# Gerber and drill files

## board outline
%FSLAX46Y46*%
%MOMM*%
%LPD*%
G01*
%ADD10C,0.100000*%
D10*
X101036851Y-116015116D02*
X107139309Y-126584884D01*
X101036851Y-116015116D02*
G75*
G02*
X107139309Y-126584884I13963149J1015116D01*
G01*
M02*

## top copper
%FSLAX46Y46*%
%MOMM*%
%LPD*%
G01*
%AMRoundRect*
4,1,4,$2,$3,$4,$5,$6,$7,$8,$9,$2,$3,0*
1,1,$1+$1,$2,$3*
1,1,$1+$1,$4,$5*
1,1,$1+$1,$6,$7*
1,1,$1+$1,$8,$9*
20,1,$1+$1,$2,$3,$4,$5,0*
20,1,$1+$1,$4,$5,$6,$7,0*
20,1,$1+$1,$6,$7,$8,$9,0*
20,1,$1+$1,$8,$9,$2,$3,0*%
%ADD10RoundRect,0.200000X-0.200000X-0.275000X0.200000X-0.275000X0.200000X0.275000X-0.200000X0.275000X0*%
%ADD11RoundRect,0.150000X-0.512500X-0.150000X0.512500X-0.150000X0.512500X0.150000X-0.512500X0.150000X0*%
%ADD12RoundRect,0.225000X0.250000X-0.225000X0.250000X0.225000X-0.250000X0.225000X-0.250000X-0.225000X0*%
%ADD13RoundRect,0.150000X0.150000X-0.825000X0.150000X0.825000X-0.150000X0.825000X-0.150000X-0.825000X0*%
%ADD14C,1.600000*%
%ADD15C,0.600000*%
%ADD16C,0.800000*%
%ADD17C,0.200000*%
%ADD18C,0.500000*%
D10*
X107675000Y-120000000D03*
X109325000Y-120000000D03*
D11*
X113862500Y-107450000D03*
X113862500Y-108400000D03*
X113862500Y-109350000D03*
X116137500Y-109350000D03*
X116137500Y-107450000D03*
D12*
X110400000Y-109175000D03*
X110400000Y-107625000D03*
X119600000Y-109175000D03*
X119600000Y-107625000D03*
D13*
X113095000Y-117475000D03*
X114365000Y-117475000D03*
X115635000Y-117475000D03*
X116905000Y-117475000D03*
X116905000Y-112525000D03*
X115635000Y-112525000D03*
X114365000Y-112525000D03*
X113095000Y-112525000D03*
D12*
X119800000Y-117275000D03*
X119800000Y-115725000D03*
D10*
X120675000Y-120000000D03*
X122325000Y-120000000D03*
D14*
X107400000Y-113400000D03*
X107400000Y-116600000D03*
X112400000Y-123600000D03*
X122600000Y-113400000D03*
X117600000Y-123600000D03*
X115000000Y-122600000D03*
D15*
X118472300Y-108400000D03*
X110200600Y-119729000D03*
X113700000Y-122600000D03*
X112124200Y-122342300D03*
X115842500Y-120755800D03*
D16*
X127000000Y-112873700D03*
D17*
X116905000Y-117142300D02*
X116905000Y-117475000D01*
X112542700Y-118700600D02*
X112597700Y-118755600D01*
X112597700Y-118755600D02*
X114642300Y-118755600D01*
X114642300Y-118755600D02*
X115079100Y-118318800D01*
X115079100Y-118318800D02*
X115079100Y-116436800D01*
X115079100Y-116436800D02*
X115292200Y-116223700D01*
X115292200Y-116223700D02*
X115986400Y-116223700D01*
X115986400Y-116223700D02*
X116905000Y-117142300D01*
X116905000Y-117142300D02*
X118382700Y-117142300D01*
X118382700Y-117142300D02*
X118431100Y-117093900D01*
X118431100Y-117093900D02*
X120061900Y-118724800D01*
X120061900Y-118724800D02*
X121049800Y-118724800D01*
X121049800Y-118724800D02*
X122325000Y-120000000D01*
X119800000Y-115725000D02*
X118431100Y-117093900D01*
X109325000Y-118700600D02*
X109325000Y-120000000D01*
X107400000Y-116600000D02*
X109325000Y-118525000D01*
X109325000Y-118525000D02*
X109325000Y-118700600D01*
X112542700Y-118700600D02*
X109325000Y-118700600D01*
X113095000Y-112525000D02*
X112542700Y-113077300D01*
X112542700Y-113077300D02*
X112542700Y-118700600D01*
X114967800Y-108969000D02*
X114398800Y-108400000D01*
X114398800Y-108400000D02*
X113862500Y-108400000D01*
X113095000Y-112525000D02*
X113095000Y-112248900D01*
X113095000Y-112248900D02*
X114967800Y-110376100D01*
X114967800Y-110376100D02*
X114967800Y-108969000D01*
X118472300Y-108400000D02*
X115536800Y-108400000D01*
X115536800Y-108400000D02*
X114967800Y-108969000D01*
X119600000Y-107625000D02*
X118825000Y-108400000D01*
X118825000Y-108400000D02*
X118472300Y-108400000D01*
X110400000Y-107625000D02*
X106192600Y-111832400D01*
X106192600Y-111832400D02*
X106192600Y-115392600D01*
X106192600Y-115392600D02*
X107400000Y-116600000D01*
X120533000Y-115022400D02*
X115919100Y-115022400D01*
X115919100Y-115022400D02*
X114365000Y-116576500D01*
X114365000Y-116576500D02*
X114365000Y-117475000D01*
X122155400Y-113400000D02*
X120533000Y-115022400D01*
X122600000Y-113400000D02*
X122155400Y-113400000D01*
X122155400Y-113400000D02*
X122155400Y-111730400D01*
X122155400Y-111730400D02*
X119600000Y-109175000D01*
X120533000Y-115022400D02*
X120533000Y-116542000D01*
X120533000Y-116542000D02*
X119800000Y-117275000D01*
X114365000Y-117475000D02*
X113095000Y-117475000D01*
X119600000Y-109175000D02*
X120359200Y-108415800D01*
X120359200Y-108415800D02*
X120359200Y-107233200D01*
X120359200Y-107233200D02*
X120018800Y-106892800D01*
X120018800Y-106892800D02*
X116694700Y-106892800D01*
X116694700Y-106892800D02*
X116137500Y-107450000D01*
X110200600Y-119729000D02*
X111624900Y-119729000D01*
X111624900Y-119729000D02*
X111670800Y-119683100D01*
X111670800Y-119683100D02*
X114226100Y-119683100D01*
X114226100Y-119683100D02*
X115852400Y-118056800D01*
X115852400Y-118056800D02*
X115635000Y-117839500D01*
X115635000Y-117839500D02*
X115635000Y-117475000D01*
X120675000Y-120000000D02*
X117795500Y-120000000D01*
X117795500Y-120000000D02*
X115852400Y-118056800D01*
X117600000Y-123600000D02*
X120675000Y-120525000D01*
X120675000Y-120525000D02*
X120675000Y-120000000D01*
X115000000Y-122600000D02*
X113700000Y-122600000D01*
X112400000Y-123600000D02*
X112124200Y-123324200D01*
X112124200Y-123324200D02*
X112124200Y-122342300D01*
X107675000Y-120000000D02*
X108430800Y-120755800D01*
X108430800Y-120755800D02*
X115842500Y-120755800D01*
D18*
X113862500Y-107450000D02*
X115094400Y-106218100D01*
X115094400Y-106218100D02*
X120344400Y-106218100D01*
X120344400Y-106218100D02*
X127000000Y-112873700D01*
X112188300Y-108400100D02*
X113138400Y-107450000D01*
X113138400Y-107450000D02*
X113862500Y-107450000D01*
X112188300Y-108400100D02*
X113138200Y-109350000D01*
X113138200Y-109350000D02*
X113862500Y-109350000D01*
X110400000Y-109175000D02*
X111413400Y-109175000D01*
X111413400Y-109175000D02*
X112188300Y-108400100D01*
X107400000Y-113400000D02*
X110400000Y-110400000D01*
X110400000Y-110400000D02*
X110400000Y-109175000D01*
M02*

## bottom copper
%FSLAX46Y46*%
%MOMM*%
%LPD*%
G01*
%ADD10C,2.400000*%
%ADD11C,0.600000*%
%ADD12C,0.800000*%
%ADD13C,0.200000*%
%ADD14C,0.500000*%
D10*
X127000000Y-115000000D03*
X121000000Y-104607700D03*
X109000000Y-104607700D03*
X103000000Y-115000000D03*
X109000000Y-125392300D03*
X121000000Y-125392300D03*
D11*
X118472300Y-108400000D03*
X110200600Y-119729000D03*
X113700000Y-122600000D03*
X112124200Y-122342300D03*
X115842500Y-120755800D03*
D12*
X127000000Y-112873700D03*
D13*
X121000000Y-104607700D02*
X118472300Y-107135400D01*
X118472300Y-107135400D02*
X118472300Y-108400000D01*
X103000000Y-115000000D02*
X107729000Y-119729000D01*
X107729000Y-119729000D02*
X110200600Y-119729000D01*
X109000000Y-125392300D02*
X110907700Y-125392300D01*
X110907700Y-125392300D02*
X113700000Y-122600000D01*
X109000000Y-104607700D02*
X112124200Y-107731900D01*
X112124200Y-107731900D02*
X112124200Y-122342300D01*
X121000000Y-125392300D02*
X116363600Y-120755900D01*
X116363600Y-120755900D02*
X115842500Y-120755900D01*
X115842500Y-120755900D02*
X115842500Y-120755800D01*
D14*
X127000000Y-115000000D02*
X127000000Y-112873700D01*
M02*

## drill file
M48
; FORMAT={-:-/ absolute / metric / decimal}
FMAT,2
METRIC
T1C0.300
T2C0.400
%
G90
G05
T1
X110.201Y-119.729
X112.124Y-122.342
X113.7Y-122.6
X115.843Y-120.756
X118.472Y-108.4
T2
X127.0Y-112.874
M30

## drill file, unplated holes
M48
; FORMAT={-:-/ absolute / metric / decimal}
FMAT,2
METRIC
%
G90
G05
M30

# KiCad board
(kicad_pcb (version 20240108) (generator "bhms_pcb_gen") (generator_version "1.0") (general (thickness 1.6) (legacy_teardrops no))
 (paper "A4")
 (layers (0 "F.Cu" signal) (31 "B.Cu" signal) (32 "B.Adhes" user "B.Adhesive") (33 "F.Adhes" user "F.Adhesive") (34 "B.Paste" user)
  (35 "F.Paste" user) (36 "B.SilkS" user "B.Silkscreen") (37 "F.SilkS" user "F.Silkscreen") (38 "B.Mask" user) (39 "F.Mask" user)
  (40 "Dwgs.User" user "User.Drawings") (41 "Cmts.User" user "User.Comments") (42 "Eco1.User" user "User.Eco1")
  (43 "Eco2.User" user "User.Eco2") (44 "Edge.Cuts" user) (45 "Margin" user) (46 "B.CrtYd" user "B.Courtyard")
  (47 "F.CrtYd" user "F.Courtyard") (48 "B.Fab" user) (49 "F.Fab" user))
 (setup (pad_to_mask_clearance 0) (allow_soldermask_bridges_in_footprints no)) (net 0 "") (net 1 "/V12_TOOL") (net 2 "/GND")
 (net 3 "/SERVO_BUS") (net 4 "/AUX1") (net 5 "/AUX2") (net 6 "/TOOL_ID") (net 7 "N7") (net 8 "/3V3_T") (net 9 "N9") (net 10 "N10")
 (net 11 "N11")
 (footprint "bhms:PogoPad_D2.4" (layer "F.Cu") (at 127 115)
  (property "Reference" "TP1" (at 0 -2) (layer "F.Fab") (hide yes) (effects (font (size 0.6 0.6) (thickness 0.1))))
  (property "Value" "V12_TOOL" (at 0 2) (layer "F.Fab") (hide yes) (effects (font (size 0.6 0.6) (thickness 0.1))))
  (pad "1" smd circle (at 0 0 0) (size 2.4 2.4) (layers "B.Cu" "B.Mask") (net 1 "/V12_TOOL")))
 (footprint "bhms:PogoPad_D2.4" (layer "F.Cu") (at 121 104.6077)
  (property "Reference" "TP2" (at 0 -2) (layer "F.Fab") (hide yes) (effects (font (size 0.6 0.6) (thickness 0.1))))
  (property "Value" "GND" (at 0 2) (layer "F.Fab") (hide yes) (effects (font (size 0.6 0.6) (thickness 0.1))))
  (pad "1" smd circle (at 0 0 0) (size 2.4 2.4) (layers "B.Cu" "B.Mask") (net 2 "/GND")))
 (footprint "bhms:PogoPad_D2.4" (layer "F.Cu") (at 109 104.6077)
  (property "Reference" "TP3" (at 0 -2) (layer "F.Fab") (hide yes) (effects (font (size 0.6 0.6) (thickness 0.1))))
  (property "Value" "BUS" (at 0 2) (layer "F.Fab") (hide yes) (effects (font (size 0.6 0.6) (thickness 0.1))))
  (pad "1" smd circle (at 0 0 0) (size 2.4 2.4) (layers "B.Cu" "B.Mask") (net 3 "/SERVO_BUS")))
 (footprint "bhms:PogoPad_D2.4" (layer "F.Cu") (at 103 115)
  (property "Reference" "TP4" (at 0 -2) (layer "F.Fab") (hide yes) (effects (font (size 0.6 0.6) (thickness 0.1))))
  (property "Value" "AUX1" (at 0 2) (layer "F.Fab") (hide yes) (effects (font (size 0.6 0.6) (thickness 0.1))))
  (pad "1" smd circle (at 0 0 0) (size 2.4 2.4) (layers "B.Cu" "B.Mask") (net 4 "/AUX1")))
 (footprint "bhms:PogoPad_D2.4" (layer "F.Cu") (at 109 125.3923)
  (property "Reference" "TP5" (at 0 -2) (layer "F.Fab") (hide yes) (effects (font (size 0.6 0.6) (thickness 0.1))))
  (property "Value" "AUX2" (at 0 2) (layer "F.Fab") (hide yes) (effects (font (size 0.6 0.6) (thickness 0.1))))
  (pad "1" smd circle (at 0 0 0) (size 2.4 2.4) (layers "B.Cu" "B.Mask") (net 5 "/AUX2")))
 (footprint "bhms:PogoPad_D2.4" (layer "F.Cu") (at 121 125.3923)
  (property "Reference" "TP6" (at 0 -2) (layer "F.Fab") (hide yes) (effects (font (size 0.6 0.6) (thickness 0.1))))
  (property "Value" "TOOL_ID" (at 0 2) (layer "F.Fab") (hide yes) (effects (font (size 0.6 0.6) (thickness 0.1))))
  (pad "1" smd circle (at 0 0 0) (size 2.4 2.4) (layers "B.Cu" "B.Mask") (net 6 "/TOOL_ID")))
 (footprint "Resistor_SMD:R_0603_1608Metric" (layer "F.Cu") (at 108.5 120)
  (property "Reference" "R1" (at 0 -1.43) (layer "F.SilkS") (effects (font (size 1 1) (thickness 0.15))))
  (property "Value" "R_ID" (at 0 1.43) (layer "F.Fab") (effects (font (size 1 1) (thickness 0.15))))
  (pad "1" smd roundrect (at -0.825 0 0) (size 0.8 0.95) (layers "F.Cu" "F.Mask" "F.Paste") (roundrect_rratio 0.25) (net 6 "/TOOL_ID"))
  (pad "2" smd roundrect (at 0.825 0 0) (size 0.8 0.95) (layers "F.Cu" "F.Mask" "F.Paste") (roundrect_rratio 0.25) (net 2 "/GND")))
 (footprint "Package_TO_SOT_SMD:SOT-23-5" (layer "F.Cu") (at 115 108.4)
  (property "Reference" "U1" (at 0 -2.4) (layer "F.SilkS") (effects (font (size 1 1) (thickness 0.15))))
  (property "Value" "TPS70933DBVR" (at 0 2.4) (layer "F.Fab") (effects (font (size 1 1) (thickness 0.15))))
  (pad "1" smd roundrect (at -1.1375 -0.95 0) (size 1.325 0.6) (layers "F.Cu" "F.Mask" "F.Paste") (roundrect_rratio 0.25)
   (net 1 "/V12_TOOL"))
  (pad "2" smd roundrect (at -1.1375 0 0) (size 1.325 0.6) (layers "F.Cu" "F.Mask" "F.Paste") (roundrect_rratio 0.25) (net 2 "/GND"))
  (pad "3" smd roundrect (at -1.1375 0.95 0) (size 1.325 0.6) (layers "F.Cu" "F.Mask" "F.Paste") (roundrect_rratio 0.25) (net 1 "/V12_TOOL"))
  (pad "4" smd roundrect (at 1.1375 0.95 0) (size 1.325 0.6) (layers "F.Cu" "F.Mask" "F.Paste") (roundrect_rratio 0.25) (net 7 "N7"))
  (pad "5" smd roundrect (at 1.1375 -0.95 0) (size 1.325 0.6) (layers "F.Cu" "F.Mask" "F.Paste") (roundrect_rratio 0.25) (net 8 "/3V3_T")))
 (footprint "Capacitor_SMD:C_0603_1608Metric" (layer "F.Cu") (at 110.4 108.4 90)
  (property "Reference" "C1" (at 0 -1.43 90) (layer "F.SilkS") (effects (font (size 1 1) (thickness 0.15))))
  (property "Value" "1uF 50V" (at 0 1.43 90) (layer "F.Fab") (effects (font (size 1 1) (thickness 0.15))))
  (pad "1" smd roundrect (at -0.775 0 90) (size 0.9 0.95) (layers "F.Cu" "F.Mask" "F.Paste") (roundrect_rratio 0.25) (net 1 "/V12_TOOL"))
  (pad "2" smd roundrect (at 0.775 0 90) (size 0.9 0.95) (layers "F.Cu" "F.Mask" "F.Paste") (roundrect_rratio 0.25) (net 2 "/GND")))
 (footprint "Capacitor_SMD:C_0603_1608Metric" (layer "F.Cu") (at 119.6 108.4 90)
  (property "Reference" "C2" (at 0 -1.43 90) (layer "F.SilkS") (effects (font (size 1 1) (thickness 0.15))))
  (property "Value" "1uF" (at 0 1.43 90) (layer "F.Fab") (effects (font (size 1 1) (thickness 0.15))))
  (pad "1" smd roundrect (at -0.775 0 90) (size 0.9 0.95) (layers "F.Cu" "F.Mask" "F.Paste") (roundrect_rratio 0.25) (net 8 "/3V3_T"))
  (pad "2" smd roundrect (at 0.775 0 90) (size 0.9 0.95) (layers "F.Cu" "F.Mask" "F.Paste") (roundrect_rratio 0.25) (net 2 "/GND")))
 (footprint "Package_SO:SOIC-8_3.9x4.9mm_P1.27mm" (layer "F.Cu") (at 115 115 90)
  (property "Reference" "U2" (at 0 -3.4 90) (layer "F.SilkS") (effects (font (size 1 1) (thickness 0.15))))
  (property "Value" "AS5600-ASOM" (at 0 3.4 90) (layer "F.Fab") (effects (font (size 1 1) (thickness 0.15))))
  (pad "1" smd roundrect (at -2.475 -1.905 90) (size 1.95 0.6) (layers "F.Cu" "F.Mask" "F.Paste") (roundrect_rratio 0.25) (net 8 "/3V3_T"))
  (pad "2" smd roundrect (at -2.475 -0.635 90) (size 1.95 0.6) (layers "F.Cu" "F.Mask" "F.Paste") (roundrect_rratio 0.25) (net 8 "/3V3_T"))
  (pad "3" smd roundrect (at -2.475 0.635 90) (size 1.95 0.6) (layers "F.Cu" "F.Mask" "F.Paste") (roundrect_rratio 0.25) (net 4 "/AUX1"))
  (pad "4" smd roundrect (at -2.475 1.905 90) (size 1.95 0.6) (layers "F.Cu" "F.Mask" "F.Paste") (roundrect_rratio 0.25) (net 2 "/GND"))
  (pad "5" smd roundrect (at 2.475 1.905 90) (size 1.95 0.6) (layers "F.Cu" "F.Mask" "F.Paste") (roundrect_rratio 0.25) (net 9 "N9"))
  (pad "6" smd roundrect (at 2.475 0.635 90) (size 1.95 0.6) (layers "F.Cu" "F.Mask" "F.Paste") (roundrect_rratio 0.25) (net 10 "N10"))
  (pad "7" smd roundrect (at 2.475 -0.635 90) (size 1.95 0.6) (layers "F.Cu" "F.Mask" "F.Paste") (roundrect_rratio 0.25) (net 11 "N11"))
  (pad "8" smd roundrect (at 2.475 -1.905 90) (size 1.95 0.6) (layers "F.Cu" "F.Mask" "F.Paste") (roundrect_rratio 0.25) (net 2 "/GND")))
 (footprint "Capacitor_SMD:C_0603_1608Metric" (layer "F.Cu") (at 119.8 116.5 90)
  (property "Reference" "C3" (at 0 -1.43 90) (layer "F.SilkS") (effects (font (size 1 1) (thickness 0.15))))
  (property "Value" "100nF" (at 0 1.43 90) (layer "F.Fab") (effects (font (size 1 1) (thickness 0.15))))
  (pad "1" smd roundrect (at -0.775 0 90) (size 0.9 0.95) (layers "F.Cu" "F.Mask" "F.Paste") (roundrect_rratio 0.25) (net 8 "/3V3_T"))
  (pad "2" smd roundrect (at 0.775 0 90) (size 0.9 0.95) (layers "F.Cu" "F.Mask" "F.Paste") (roundrect_rratio 0.25) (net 2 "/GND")))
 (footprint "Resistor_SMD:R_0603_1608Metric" (layer "F.Cu") (at 121.5 120)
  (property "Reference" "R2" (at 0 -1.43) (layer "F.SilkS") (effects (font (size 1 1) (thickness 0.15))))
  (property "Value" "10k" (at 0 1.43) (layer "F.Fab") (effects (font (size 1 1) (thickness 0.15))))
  (pad "1" smd roundrect (at -0.825 0 0) (size 0.8 0.95) (layers "F.Cu" "F.Mask" "F.Paste") (roundrect_rratio 0.25) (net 4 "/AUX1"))
  (pad "2" smd roundrect (at 0.825 0 0) (size 0.8 0.95) (layers "F.Cu" "F.Mask" "F.Paste") (roundrect_rratio 0.25) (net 2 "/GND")))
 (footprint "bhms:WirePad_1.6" (layer "F.Cu") (at 107.4 113.4)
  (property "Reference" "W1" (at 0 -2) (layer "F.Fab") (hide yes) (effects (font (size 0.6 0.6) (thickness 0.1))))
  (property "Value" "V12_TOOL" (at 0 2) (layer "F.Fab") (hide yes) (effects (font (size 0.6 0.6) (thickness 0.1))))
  (pad "1" smd circle (at 0 0 0) (size 1.6 1.6) (layers "F.Cu" "F.Mask") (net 1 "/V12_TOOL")))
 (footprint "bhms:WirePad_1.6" (layer "F.Cu") (at 107.4 116.6)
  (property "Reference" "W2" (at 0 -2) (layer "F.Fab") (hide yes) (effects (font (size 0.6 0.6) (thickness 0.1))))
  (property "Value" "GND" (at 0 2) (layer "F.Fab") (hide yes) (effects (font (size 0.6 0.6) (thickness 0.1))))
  (pad "1" smd circle (at 0 0 0) (size 1.6 1.6) (layers "F.Cu" "F.Mask") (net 2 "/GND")))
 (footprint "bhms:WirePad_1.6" (layer "F.Cu") (at 112.4 123.6)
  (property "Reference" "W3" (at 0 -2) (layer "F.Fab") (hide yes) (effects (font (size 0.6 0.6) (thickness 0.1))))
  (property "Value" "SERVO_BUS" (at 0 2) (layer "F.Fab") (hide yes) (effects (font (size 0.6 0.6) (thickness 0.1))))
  (pad "1" smd circle (at 0 0 0) (size 1.6 1.6) (layers "F.Cu" "F.Mask") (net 3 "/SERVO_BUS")))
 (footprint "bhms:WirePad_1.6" (layer "F.Cu") (at 122.6 113.4)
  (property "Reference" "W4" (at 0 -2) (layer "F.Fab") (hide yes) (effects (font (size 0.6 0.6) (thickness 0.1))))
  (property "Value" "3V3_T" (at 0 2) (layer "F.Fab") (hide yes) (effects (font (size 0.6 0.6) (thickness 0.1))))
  (pad "1" smd circle (at 0 0 0) (size 1.6 1.6) (layers "F.Cu" "F.Mask") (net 8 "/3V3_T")))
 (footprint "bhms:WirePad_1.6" (layer "F.Cu") (at 117.6 123.6)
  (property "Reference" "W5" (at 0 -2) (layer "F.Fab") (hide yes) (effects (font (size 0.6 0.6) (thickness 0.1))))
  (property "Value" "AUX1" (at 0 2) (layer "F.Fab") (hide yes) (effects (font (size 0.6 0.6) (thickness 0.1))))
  (pad "1" smd circle (at 0 0 0) (size 1.6 1.6) (layers "F.Cu" "F.Mask") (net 4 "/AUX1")))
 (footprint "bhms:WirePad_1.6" (layer "F.Cu") (at 115 122.6)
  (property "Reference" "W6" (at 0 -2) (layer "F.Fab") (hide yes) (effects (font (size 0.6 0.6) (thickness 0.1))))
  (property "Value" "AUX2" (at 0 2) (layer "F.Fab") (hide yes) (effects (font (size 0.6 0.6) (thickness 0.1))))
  (pad "1" smd circle (at 0 0 0) (size 1.6 1.6) (layers "F.Cu" "F.Mask") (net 5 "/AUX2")))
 (gr_line (start 101.036851 116.015116) (end 107.139309 126.584884) (stroke (width 0.1) (type default)) (layer "Edge.Cuts"))
 (gr_arc (start 107.139309 126.584884) (mid 127.124356 108) (end 101.036851 116.015116) (stroke (width 0.1) (type default))
  (layer "Edge.Cuts"))
 (segment (start 116.905 117.1423) (end 116.905 117.475) (width 0.2) (layer "F.Cu") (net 2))
 (segment (start 112.5427 118.7006) (end 112.5977 118.7556) (width 0.2) (layer "F.Cu") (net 2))
 (segment (start 112.5977 118.7556) (end 114.6423 118.7556) (width 0.2) (layer "F.Cu") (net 2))
 (segment (start 114.6423 118.7556) (end 115.0791 118.3188) (width 0.2) (layer "F.Cu") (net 2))
 (segment (start 115.0791 118.3188) (end 115.0791 116.4368) (width 0.2) (layer "F.Cu") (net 2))
 (segment (start 115.0791 116.4368) (end 115.2922 116.2237) (width 0.2) (layer "F.Cu") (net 2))
 (segment (start 115.2922 116.2237) (end 115.9864 116.2237) (width 0.2) (layer "F.Cu") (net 2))
 (segment (start 115.9864 116.2237) (end 116.905 117.1423) (width 0.2) (layer "F.Cu") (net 2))
 (segment (start 116.905 117.1423) (end 118.3827 117.1423) (width 0.2) (layer "F.Cu") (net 2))
 (segment (start 118.3827 117.1423) (end 118.4311 117.0939) (width 0.2) (layer "F.Cu") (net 2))
 (segment (start 118.4311 117.0939) (end 120.0619 118.7248) (width 0.2) (layer "F.Cu") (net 2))
 (segment (start 120.0619 118.7248) (end 121.0498 118.7248) (width 0.2) (layer "F.Cu") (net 2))
 (segment (start 121.0498 118.7248) (end 122.325 120) (width 0.2) (layer "F.Cu") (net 2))
 (segment (start 119.8 115.725) (end 118.4311 117.0939) (width 0.2) (layer "F.Cu") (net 2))
 (segment (start 109.325 118.7006) (end 109.325 120) (width 0.2) (layer "F.Cu") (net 2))
 (segment (start 107.4 116.6) (end 109.325 118.525) (width 0.2) (layer "F.Cu") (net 2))
 (segment (start 109.325 118.525) (end 109.325 118.7006) (width 0.2) (layer "F.Cu") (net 2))
 (segment (start 112.5427 118.7006) (end 109.325 118.7006) (width 0.2) (layer "F.Cu") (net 2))
 (segment (start 113.095 112.525) (end 112.5427 113.0773) (width 0.2) (layer "F.Cu") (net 2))
 (segment (start 112.5427 113.0773) (end 112.5427 118.7006) (width 0.2) (layer "F.Cu") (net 2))
 (segment (start 114.9678 108.969) (end 114.3988 108.4) (width 0.2) (layer "F.Cu") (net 2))
 (segment (start 114.3988 108.4) (end 113.8625 108.4) (width 0.2) (layer "F.Cu") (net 2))
 (segment (start 113.095 112.525) (end 113.095 112.2489) (width 0.2) (layer "F.Cu") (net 2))
 (segment (start 113.095 112.2489) (end 114.9678 110.3761) (width 0.2) (layer "F.Cu") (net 2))
 (segment (start 114.9678 110.3761) (end 114.9678 108.969) (width 0.2) (layer "F.Cu") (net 2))
 (segment (start 118.4723 108.4) (end 115.5368 108.4) (width 0.2) (layer "F.Cu") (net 2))
 (segment (start 115.5368 108.4) (end 114.9678 108.969) (width 0.2) (layer "F.Cu") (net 2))
 (segment (start 119.6 107.625) (end 118.825 108.4) (width 0.2) (layer "F.Cu") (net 2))
 (segment (start 118.825 108.4) (end 118.4723 108.4) (width 0.2) (layer "F.Cu") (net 2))
 (segment (start 110.4 107.625) (end 106.1926 111.8324) (width 0.2) (layer "F.Cu") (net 2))
 (segment (start 106.1926 111.8324) (end 106.1926 115.3926) (width 0.2) (layer "F.Cu") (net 2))
 (segment (start 106.1926 115.3926) (end 107.4 116.6) (width 0.2) (layer "F.Cu") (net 2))
 (segment (start 121 104.6077) (end 118.4723 107.1354) (width 0.2) (layer "B.Cu") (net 2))
 (segment (start 118.4723 107.1354) (end 118.4723 108.4) (width 0.2) (layer "B.Cu") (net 2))
 (segment (start 120.533 115.0224) (end 115.9191 115.0224) (width 0.2) (layer "F.Cu") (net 8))
 (segment (start 115.9191 115.0224) (end 114.365 116.5765) (width 0.2) (layer "F.Cu") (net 8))
 (segment (start 114.365 116.5765) (end 114.365 117.475) (width 0.2) (layer "F.Cu") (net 8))
 (segment (start 122.1554 113.4) (end 120.533 115.0224) (width 0.2) (layer "F.Cu") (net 8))
 (segment (start 122.6 113.4) (end 122.1554 113.4) (width 0.2) (layer "F.Cu") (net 8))
 (segment (start 122.1554 113.4) (end 122.1554 111.7304) (width 0.2) (layer "F.Cu") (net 8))
 (segment (start 122.1554 111.7304) (end 119.6 109.175) (width 0.2) (layer "F.Cu") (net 8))
 (segment (start 120.533 115.0224) (end 120.533 116.542) (width 0.2) (layer "F.Cu") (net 8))
 (segment (start 120.533 116.542) (end 119.8 117.275) (width 0.2) (layer "F.Cu") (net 8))
 (segment (start 114.365 117.475) (end 113.095 117.475) (width 0.2) (layer "F.Cu") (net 8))
 (segment (start 119.6 109.175) (end 120.3592 108.4158) (width 0.2) (layer "F.Cu") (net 8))
 (segment (start 120.3592 108.4158) (end 120.3592 107.2332) (width 0.2) (layer "F.Cu") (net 8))
 (segment (start 120.3592 107.2332) (end 120.0188 106.8928) (width 0.2) (layer "F.Cu") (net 8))
 (segment (start 120.0188 106.8928) (end 116.6947 106.8928) (width 0.2) (layer "F.Cu") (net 8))
 (segment (start 116.6947 106.8928) (end 116.1375 107.45) (width 0.2) (layer "F.Cu") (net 8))
 (segment (start 110.2006 119.729) (end 111.6249 119.729) (width 0.2) (layer "F.Cu") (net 4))
 (segment (start 111.6249 119.729) (end 111.6708 119.6831) (width 0.2) (layer "F.Cu") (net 4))
 (segment (start 111.6708 119.6831) (end 114.2261 119.6831) (width 0.2) (layer "F.Cu") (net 4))
 (segment (start 114.2261 119.6831) (end 115.8524 118.0568) (width 0.2) (layer "F.Cu") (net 4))
 (segment (start 103 115) (end 107.729 119.729) (width 0.2) (layer "B.Cu") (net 4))
 (segment (start 107.729 119.729) (end 110.2006 119.729) (width 0.2) (layer "B.Cu") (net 4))
 (segment (start 115.8524 118.0568) (end 115.635 117.8395) (width 0.2) (layer "F.Cu") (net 4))
 (segment (start 115.635 117.8395) (end 115.635 117.475) (width 0.2) (layer "F.Cu") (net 4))
 (segment (start 120.675 120) (end 117.7955 120) (width 0.2) (layer "F.Cu") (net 4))
 (segment (start 117.7955 120) (end 115.8524 118.0568) (width 0.2) (layer "F.Cu") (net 4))
 (segment (start 117.6 123.6) (end 120.675 120.525) (width 0.2) (layer "F.Cu") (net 4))
 (segment (start 120.675 120.525) (end 120.675 120) (width 0.2) (layer "F.Cu") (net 4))
 (segment (start 115 122.6) (end 113.7 122.6) (width 0.2) (layer "F.Cu") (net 5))
 (segment (start 109 125.3923) (end 110.9077 125.3923) (width 0.2) (layer "B.Cu") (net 5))
 (segment (start 110.9077 125.3923) (end 113.7 122.6) (width 0.2) (layer "B.Cu") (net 5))
 (segment (start 112.4 123.6) (end 112.1242 123.3242) (width 0.2) (layer "F.Cu") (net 3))
 (segment (start 112.1242 123.3242) (end 112.1242 122.3423) (width 0.2) (layer "F.Cu") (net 3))
 (segment (start 109 104.6077) (end 112.1242 107.7319) (width 0.2) (layer "B.Cu") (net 3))
 (segment (start 112.1242 107.7319) (end 112.1242 122.3423) (width 0.2) (layer "B.Cu") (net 3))
 (segment (start 107.675 120) (end 108.4308 120.7558) (width 0.2) (layer "F.Cu") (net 6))
 (segment (start 108.4308 120.7558) (end 115.8425 120.7558) (width 0.2) (layer "F.Cu") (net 6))
 (segment (start 121 125.3923) (end 116.3636 120.7559) (width 0.2) (layer "B.Cu") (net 6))
 (segment (start 116.3636 120.7559) (end 115.8425 120.7559) (width 0.2) (layer "B.Cu") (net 6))
 (segment (start 115.8425 120.7559) (end 115.8425 120.7558) (width 0.2) (layer "B.Cu") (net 6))
 (segment (start 113.8625 107.45) (end 115.0944 106.2181) (width 0.5) (layer "F.Cu") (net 1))
 (segment (start 115.0944 106.2181) (end 120.3444 106.2181) (width 0.5) (layer "F.Cu") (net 1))
 (segment (start 120.3444 106.2181) (end 127 112.8737) (width 0.5) (layer "F.Cu") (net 1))
 (segment (start 112.1883 108.4001) (end 113.1384 107.45) (width 0.5) (layer "F.Cu") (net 1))
 (segment (start 113.1384 107.45) (end 113.8625 107.45) (width 0.5) (layer "F.Cu") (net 1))
 (segment (start 127 115) (end 127 112.8737) (width 0.5) (layer "B.Cu") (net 1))
 (segment (start 112.1883 108.4001) (end 113.1382 109.35) (width 0.5) (layer "F.Cu") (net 1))
 (segment (start 113.1382 109.35) (end 113.8625 109.35) (width 0.5) (layer "F.Cu") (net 1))
 (segment (start 110.4 109.175) (end 111.4134 109.175) (width 0.5) (layer "F.Cu") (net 1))
 (segment (start 111.4134 109.175) (end 112.1883 108.4001) (width 0.5) (layer "F.Cu") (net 1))
 (segment (start 107.4 113.4) (end 110.4 110.4) (width 0.5) (layer "F.Cu") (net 1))
 (segment (start 110.4 110.4) (end 110.4 109.175) (width 0.5) (layer "F.Cu") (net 1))
 (via (at 118.4723 108.4) (size 0.6) (drill 0.3) (layers "F.Cu" "B.Cu") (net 2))
 (via (at 110.2006 119.729) (size 0.6) (drill 0.3) (layers "F.Cu" "B.Cu") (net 4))
 (via (at 113.7 122.6) (size 0.6) (drill 0.3) (layers "F.Cu" "B.Cu") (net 5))
 (via (at 112.1242 122.3423) (size 0.6) (drill 0.3) (layers "F.Cu" "B.Cu") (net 3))
 (via (at 115.8425 120.7558) (size 0.6) (drill 0.3) (layers "F.Cu" "B.Cu") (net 6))
 (via (at 127 112.8737) (size 0.8) (drill 0.4) (layers "F.Cu" "B.Cu") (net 1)))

